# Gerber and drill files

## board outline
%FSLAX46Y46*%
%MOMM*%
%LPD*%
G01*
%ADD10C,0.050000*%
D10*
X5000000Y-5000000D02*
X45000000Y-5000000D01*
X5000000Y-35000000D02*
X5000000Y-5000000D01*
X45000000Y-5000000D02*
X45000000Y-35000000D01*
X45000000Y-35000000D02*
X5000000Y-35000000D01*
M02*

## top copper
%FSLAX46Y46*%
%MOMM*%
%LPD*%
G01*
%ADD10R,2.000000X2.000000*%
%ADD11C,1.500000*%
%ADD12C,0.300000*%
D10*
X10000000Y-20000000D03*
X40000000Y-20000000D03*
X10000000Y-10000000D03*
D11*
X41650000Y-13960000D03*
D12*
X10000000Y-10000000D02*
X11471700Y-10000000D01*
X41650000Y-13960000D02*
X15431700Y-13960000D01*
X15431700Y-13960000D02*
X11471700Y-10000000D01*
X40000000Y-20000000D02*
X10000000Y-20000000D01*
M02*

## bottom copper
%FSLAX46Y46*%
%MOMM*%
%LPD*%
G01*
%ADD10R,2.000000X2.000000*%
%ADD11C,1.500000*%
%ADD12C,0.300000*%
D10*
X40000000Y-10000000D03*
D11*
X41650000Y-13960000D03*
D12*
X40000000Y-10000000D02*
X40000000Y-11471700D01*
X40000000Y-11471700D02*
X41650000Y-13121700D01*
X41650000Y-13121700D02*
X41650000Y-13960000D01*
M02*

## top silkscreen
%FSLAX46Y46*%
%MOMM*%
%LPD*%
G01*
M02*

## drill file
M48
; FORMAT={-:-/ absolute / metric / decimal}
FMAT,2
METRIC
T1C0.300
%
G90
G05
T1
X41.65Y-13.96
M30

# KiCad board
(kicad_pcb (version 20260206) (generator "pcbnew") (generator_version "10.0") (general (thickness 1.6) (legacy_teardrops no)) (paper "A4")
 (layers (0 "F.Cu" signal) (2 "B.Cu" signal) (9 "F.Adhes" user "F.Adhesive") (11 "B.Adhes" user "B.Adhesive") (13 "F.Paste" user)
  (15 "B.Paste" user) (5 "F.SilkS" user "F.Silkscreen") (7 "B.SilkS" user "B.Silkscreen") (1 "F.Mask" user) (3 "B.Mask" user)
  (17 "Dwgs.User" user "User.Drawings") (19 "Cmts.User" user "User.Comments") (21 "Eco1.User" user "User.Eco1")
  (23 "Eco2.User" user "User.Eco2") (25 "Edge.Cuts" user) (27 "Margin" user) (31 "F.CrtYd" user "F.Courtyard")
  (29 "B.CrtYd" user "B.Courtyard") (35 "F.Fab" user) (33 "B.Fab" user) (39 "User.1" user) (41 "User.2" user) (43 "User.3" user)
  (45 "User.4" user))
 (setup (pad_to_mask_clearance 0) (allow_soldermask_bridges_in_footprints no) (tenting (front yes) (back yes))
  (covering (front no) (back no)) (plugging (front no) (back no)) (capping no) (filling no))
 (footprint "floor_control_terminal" (layer "F.Cu") (at 10 20)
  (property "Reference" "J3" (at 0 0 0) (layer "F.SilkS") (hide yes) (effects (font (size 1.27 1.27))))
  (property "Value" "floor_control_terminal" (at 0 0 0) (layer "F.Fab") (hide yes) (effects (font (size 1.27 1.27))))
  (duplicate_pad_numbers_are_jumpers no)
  (pad "1" smd rect (at 0 0) (size 2 2) (layers "F.Cu" "F.Mask" "F.Paste") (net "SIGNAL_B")))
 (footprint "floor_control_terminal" (layer "F.Cu") (at 40 20)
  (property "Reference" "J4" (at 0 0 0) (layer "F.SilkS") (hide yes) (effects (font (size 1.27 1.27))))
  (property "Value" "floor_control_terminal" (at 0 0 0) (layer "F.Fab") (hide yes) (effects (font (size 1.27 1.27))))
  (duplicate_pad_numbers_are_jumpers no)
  (pad "1" smd rect (at 0 0) (size 2 2) (layers "F.Cu" "F.Mask" "F.Paste") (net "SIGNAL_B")))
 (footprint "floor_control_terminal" (layer "F.Cu") (at 10 10)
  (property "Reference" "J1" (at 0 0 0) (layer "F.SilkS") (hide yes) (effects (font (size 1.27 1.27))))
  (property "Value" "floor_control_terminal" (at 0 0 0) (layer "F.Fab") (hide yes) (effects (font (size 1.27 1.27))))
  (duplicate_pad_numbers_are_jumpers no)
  (pad "1" smd rect (at 0 0) (size 2 2) (layers "F.Cu" "F.Mask" "F.Paste") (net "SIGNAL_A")))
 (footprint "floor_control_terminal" (layer "B.Cu") (at 40 10)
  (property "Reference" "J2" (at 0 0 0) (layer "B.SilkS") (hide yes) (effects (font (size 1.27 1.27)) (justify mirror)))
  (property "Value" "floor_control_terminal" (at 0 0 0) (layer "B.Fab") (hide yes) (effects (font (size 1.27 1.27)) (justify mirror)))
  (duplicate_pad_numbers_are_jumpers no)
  (pad "1" smd rect (at 0 0) (size 2 2) (layers "B.Cu" "B.Mask" "B.Paste") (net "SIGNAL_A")))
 (gr_line (start 5 5) (end 45 5) (stroke (width 0.05) (type default)) (layer "Edge.Cuts"))
 (gr_line (start 5 35) (end 5 5) (stroke (width 0.05) (type default)) (layer "Edge.Cuts"))
 (gr_line (start 45 5) (end 45 35) (stroke (width 0.05) (type default)) (layer "Edge.Cuts"))
 (gr_line (start 45 35) (end 5 35) (stroke (width 0.05) (type default)) (layer "Edge.Cuts"))
 (segment (start 10 10) (end 11.4717 10) (width 0.3) (layer "F.Cu") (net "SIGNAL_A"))
 (segment (start 41.65 13.96) (end 15.4317 13.96) (width 0.3) (layer "F.Cu") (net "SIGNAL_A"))
 (segment (start 15.4317 13.96) (end 11.4717 10) (width 0.3) (layer "F.Cu") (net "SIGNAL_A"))
 (via (at 41.65 13.96) (size 1.5) (drill 0.3) (layers "F.Cu" "B.Cu") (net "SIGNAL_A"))
 (segment (start 40 10) (end 40 11.4717) (width 0.3) (layer "B.Cu") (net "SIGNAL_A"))
 (segment (start 40 11.4717) (end 41.65 13.1217) (width 0.3) (layer "B.Cu") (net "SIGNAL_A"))
 (segment (start 41.65 13.1217) (end 41.65 13.96) (width 0.3) (layer "B.Cu") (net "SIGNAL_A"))
 (segment (start 40 20) (end 10 20) (width 0.3) (layer "F.Cu") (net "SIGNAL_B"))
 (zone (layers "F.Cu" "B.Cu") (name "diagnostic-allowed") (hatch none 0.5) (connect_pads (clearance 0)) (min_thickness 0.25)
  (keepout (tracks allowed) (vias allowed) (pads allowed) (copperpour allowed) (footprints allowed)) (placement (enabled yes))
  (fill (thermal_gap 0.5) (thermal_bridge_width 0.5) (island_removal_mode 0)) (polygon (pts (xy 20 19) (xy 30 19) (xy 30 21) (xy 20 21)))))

